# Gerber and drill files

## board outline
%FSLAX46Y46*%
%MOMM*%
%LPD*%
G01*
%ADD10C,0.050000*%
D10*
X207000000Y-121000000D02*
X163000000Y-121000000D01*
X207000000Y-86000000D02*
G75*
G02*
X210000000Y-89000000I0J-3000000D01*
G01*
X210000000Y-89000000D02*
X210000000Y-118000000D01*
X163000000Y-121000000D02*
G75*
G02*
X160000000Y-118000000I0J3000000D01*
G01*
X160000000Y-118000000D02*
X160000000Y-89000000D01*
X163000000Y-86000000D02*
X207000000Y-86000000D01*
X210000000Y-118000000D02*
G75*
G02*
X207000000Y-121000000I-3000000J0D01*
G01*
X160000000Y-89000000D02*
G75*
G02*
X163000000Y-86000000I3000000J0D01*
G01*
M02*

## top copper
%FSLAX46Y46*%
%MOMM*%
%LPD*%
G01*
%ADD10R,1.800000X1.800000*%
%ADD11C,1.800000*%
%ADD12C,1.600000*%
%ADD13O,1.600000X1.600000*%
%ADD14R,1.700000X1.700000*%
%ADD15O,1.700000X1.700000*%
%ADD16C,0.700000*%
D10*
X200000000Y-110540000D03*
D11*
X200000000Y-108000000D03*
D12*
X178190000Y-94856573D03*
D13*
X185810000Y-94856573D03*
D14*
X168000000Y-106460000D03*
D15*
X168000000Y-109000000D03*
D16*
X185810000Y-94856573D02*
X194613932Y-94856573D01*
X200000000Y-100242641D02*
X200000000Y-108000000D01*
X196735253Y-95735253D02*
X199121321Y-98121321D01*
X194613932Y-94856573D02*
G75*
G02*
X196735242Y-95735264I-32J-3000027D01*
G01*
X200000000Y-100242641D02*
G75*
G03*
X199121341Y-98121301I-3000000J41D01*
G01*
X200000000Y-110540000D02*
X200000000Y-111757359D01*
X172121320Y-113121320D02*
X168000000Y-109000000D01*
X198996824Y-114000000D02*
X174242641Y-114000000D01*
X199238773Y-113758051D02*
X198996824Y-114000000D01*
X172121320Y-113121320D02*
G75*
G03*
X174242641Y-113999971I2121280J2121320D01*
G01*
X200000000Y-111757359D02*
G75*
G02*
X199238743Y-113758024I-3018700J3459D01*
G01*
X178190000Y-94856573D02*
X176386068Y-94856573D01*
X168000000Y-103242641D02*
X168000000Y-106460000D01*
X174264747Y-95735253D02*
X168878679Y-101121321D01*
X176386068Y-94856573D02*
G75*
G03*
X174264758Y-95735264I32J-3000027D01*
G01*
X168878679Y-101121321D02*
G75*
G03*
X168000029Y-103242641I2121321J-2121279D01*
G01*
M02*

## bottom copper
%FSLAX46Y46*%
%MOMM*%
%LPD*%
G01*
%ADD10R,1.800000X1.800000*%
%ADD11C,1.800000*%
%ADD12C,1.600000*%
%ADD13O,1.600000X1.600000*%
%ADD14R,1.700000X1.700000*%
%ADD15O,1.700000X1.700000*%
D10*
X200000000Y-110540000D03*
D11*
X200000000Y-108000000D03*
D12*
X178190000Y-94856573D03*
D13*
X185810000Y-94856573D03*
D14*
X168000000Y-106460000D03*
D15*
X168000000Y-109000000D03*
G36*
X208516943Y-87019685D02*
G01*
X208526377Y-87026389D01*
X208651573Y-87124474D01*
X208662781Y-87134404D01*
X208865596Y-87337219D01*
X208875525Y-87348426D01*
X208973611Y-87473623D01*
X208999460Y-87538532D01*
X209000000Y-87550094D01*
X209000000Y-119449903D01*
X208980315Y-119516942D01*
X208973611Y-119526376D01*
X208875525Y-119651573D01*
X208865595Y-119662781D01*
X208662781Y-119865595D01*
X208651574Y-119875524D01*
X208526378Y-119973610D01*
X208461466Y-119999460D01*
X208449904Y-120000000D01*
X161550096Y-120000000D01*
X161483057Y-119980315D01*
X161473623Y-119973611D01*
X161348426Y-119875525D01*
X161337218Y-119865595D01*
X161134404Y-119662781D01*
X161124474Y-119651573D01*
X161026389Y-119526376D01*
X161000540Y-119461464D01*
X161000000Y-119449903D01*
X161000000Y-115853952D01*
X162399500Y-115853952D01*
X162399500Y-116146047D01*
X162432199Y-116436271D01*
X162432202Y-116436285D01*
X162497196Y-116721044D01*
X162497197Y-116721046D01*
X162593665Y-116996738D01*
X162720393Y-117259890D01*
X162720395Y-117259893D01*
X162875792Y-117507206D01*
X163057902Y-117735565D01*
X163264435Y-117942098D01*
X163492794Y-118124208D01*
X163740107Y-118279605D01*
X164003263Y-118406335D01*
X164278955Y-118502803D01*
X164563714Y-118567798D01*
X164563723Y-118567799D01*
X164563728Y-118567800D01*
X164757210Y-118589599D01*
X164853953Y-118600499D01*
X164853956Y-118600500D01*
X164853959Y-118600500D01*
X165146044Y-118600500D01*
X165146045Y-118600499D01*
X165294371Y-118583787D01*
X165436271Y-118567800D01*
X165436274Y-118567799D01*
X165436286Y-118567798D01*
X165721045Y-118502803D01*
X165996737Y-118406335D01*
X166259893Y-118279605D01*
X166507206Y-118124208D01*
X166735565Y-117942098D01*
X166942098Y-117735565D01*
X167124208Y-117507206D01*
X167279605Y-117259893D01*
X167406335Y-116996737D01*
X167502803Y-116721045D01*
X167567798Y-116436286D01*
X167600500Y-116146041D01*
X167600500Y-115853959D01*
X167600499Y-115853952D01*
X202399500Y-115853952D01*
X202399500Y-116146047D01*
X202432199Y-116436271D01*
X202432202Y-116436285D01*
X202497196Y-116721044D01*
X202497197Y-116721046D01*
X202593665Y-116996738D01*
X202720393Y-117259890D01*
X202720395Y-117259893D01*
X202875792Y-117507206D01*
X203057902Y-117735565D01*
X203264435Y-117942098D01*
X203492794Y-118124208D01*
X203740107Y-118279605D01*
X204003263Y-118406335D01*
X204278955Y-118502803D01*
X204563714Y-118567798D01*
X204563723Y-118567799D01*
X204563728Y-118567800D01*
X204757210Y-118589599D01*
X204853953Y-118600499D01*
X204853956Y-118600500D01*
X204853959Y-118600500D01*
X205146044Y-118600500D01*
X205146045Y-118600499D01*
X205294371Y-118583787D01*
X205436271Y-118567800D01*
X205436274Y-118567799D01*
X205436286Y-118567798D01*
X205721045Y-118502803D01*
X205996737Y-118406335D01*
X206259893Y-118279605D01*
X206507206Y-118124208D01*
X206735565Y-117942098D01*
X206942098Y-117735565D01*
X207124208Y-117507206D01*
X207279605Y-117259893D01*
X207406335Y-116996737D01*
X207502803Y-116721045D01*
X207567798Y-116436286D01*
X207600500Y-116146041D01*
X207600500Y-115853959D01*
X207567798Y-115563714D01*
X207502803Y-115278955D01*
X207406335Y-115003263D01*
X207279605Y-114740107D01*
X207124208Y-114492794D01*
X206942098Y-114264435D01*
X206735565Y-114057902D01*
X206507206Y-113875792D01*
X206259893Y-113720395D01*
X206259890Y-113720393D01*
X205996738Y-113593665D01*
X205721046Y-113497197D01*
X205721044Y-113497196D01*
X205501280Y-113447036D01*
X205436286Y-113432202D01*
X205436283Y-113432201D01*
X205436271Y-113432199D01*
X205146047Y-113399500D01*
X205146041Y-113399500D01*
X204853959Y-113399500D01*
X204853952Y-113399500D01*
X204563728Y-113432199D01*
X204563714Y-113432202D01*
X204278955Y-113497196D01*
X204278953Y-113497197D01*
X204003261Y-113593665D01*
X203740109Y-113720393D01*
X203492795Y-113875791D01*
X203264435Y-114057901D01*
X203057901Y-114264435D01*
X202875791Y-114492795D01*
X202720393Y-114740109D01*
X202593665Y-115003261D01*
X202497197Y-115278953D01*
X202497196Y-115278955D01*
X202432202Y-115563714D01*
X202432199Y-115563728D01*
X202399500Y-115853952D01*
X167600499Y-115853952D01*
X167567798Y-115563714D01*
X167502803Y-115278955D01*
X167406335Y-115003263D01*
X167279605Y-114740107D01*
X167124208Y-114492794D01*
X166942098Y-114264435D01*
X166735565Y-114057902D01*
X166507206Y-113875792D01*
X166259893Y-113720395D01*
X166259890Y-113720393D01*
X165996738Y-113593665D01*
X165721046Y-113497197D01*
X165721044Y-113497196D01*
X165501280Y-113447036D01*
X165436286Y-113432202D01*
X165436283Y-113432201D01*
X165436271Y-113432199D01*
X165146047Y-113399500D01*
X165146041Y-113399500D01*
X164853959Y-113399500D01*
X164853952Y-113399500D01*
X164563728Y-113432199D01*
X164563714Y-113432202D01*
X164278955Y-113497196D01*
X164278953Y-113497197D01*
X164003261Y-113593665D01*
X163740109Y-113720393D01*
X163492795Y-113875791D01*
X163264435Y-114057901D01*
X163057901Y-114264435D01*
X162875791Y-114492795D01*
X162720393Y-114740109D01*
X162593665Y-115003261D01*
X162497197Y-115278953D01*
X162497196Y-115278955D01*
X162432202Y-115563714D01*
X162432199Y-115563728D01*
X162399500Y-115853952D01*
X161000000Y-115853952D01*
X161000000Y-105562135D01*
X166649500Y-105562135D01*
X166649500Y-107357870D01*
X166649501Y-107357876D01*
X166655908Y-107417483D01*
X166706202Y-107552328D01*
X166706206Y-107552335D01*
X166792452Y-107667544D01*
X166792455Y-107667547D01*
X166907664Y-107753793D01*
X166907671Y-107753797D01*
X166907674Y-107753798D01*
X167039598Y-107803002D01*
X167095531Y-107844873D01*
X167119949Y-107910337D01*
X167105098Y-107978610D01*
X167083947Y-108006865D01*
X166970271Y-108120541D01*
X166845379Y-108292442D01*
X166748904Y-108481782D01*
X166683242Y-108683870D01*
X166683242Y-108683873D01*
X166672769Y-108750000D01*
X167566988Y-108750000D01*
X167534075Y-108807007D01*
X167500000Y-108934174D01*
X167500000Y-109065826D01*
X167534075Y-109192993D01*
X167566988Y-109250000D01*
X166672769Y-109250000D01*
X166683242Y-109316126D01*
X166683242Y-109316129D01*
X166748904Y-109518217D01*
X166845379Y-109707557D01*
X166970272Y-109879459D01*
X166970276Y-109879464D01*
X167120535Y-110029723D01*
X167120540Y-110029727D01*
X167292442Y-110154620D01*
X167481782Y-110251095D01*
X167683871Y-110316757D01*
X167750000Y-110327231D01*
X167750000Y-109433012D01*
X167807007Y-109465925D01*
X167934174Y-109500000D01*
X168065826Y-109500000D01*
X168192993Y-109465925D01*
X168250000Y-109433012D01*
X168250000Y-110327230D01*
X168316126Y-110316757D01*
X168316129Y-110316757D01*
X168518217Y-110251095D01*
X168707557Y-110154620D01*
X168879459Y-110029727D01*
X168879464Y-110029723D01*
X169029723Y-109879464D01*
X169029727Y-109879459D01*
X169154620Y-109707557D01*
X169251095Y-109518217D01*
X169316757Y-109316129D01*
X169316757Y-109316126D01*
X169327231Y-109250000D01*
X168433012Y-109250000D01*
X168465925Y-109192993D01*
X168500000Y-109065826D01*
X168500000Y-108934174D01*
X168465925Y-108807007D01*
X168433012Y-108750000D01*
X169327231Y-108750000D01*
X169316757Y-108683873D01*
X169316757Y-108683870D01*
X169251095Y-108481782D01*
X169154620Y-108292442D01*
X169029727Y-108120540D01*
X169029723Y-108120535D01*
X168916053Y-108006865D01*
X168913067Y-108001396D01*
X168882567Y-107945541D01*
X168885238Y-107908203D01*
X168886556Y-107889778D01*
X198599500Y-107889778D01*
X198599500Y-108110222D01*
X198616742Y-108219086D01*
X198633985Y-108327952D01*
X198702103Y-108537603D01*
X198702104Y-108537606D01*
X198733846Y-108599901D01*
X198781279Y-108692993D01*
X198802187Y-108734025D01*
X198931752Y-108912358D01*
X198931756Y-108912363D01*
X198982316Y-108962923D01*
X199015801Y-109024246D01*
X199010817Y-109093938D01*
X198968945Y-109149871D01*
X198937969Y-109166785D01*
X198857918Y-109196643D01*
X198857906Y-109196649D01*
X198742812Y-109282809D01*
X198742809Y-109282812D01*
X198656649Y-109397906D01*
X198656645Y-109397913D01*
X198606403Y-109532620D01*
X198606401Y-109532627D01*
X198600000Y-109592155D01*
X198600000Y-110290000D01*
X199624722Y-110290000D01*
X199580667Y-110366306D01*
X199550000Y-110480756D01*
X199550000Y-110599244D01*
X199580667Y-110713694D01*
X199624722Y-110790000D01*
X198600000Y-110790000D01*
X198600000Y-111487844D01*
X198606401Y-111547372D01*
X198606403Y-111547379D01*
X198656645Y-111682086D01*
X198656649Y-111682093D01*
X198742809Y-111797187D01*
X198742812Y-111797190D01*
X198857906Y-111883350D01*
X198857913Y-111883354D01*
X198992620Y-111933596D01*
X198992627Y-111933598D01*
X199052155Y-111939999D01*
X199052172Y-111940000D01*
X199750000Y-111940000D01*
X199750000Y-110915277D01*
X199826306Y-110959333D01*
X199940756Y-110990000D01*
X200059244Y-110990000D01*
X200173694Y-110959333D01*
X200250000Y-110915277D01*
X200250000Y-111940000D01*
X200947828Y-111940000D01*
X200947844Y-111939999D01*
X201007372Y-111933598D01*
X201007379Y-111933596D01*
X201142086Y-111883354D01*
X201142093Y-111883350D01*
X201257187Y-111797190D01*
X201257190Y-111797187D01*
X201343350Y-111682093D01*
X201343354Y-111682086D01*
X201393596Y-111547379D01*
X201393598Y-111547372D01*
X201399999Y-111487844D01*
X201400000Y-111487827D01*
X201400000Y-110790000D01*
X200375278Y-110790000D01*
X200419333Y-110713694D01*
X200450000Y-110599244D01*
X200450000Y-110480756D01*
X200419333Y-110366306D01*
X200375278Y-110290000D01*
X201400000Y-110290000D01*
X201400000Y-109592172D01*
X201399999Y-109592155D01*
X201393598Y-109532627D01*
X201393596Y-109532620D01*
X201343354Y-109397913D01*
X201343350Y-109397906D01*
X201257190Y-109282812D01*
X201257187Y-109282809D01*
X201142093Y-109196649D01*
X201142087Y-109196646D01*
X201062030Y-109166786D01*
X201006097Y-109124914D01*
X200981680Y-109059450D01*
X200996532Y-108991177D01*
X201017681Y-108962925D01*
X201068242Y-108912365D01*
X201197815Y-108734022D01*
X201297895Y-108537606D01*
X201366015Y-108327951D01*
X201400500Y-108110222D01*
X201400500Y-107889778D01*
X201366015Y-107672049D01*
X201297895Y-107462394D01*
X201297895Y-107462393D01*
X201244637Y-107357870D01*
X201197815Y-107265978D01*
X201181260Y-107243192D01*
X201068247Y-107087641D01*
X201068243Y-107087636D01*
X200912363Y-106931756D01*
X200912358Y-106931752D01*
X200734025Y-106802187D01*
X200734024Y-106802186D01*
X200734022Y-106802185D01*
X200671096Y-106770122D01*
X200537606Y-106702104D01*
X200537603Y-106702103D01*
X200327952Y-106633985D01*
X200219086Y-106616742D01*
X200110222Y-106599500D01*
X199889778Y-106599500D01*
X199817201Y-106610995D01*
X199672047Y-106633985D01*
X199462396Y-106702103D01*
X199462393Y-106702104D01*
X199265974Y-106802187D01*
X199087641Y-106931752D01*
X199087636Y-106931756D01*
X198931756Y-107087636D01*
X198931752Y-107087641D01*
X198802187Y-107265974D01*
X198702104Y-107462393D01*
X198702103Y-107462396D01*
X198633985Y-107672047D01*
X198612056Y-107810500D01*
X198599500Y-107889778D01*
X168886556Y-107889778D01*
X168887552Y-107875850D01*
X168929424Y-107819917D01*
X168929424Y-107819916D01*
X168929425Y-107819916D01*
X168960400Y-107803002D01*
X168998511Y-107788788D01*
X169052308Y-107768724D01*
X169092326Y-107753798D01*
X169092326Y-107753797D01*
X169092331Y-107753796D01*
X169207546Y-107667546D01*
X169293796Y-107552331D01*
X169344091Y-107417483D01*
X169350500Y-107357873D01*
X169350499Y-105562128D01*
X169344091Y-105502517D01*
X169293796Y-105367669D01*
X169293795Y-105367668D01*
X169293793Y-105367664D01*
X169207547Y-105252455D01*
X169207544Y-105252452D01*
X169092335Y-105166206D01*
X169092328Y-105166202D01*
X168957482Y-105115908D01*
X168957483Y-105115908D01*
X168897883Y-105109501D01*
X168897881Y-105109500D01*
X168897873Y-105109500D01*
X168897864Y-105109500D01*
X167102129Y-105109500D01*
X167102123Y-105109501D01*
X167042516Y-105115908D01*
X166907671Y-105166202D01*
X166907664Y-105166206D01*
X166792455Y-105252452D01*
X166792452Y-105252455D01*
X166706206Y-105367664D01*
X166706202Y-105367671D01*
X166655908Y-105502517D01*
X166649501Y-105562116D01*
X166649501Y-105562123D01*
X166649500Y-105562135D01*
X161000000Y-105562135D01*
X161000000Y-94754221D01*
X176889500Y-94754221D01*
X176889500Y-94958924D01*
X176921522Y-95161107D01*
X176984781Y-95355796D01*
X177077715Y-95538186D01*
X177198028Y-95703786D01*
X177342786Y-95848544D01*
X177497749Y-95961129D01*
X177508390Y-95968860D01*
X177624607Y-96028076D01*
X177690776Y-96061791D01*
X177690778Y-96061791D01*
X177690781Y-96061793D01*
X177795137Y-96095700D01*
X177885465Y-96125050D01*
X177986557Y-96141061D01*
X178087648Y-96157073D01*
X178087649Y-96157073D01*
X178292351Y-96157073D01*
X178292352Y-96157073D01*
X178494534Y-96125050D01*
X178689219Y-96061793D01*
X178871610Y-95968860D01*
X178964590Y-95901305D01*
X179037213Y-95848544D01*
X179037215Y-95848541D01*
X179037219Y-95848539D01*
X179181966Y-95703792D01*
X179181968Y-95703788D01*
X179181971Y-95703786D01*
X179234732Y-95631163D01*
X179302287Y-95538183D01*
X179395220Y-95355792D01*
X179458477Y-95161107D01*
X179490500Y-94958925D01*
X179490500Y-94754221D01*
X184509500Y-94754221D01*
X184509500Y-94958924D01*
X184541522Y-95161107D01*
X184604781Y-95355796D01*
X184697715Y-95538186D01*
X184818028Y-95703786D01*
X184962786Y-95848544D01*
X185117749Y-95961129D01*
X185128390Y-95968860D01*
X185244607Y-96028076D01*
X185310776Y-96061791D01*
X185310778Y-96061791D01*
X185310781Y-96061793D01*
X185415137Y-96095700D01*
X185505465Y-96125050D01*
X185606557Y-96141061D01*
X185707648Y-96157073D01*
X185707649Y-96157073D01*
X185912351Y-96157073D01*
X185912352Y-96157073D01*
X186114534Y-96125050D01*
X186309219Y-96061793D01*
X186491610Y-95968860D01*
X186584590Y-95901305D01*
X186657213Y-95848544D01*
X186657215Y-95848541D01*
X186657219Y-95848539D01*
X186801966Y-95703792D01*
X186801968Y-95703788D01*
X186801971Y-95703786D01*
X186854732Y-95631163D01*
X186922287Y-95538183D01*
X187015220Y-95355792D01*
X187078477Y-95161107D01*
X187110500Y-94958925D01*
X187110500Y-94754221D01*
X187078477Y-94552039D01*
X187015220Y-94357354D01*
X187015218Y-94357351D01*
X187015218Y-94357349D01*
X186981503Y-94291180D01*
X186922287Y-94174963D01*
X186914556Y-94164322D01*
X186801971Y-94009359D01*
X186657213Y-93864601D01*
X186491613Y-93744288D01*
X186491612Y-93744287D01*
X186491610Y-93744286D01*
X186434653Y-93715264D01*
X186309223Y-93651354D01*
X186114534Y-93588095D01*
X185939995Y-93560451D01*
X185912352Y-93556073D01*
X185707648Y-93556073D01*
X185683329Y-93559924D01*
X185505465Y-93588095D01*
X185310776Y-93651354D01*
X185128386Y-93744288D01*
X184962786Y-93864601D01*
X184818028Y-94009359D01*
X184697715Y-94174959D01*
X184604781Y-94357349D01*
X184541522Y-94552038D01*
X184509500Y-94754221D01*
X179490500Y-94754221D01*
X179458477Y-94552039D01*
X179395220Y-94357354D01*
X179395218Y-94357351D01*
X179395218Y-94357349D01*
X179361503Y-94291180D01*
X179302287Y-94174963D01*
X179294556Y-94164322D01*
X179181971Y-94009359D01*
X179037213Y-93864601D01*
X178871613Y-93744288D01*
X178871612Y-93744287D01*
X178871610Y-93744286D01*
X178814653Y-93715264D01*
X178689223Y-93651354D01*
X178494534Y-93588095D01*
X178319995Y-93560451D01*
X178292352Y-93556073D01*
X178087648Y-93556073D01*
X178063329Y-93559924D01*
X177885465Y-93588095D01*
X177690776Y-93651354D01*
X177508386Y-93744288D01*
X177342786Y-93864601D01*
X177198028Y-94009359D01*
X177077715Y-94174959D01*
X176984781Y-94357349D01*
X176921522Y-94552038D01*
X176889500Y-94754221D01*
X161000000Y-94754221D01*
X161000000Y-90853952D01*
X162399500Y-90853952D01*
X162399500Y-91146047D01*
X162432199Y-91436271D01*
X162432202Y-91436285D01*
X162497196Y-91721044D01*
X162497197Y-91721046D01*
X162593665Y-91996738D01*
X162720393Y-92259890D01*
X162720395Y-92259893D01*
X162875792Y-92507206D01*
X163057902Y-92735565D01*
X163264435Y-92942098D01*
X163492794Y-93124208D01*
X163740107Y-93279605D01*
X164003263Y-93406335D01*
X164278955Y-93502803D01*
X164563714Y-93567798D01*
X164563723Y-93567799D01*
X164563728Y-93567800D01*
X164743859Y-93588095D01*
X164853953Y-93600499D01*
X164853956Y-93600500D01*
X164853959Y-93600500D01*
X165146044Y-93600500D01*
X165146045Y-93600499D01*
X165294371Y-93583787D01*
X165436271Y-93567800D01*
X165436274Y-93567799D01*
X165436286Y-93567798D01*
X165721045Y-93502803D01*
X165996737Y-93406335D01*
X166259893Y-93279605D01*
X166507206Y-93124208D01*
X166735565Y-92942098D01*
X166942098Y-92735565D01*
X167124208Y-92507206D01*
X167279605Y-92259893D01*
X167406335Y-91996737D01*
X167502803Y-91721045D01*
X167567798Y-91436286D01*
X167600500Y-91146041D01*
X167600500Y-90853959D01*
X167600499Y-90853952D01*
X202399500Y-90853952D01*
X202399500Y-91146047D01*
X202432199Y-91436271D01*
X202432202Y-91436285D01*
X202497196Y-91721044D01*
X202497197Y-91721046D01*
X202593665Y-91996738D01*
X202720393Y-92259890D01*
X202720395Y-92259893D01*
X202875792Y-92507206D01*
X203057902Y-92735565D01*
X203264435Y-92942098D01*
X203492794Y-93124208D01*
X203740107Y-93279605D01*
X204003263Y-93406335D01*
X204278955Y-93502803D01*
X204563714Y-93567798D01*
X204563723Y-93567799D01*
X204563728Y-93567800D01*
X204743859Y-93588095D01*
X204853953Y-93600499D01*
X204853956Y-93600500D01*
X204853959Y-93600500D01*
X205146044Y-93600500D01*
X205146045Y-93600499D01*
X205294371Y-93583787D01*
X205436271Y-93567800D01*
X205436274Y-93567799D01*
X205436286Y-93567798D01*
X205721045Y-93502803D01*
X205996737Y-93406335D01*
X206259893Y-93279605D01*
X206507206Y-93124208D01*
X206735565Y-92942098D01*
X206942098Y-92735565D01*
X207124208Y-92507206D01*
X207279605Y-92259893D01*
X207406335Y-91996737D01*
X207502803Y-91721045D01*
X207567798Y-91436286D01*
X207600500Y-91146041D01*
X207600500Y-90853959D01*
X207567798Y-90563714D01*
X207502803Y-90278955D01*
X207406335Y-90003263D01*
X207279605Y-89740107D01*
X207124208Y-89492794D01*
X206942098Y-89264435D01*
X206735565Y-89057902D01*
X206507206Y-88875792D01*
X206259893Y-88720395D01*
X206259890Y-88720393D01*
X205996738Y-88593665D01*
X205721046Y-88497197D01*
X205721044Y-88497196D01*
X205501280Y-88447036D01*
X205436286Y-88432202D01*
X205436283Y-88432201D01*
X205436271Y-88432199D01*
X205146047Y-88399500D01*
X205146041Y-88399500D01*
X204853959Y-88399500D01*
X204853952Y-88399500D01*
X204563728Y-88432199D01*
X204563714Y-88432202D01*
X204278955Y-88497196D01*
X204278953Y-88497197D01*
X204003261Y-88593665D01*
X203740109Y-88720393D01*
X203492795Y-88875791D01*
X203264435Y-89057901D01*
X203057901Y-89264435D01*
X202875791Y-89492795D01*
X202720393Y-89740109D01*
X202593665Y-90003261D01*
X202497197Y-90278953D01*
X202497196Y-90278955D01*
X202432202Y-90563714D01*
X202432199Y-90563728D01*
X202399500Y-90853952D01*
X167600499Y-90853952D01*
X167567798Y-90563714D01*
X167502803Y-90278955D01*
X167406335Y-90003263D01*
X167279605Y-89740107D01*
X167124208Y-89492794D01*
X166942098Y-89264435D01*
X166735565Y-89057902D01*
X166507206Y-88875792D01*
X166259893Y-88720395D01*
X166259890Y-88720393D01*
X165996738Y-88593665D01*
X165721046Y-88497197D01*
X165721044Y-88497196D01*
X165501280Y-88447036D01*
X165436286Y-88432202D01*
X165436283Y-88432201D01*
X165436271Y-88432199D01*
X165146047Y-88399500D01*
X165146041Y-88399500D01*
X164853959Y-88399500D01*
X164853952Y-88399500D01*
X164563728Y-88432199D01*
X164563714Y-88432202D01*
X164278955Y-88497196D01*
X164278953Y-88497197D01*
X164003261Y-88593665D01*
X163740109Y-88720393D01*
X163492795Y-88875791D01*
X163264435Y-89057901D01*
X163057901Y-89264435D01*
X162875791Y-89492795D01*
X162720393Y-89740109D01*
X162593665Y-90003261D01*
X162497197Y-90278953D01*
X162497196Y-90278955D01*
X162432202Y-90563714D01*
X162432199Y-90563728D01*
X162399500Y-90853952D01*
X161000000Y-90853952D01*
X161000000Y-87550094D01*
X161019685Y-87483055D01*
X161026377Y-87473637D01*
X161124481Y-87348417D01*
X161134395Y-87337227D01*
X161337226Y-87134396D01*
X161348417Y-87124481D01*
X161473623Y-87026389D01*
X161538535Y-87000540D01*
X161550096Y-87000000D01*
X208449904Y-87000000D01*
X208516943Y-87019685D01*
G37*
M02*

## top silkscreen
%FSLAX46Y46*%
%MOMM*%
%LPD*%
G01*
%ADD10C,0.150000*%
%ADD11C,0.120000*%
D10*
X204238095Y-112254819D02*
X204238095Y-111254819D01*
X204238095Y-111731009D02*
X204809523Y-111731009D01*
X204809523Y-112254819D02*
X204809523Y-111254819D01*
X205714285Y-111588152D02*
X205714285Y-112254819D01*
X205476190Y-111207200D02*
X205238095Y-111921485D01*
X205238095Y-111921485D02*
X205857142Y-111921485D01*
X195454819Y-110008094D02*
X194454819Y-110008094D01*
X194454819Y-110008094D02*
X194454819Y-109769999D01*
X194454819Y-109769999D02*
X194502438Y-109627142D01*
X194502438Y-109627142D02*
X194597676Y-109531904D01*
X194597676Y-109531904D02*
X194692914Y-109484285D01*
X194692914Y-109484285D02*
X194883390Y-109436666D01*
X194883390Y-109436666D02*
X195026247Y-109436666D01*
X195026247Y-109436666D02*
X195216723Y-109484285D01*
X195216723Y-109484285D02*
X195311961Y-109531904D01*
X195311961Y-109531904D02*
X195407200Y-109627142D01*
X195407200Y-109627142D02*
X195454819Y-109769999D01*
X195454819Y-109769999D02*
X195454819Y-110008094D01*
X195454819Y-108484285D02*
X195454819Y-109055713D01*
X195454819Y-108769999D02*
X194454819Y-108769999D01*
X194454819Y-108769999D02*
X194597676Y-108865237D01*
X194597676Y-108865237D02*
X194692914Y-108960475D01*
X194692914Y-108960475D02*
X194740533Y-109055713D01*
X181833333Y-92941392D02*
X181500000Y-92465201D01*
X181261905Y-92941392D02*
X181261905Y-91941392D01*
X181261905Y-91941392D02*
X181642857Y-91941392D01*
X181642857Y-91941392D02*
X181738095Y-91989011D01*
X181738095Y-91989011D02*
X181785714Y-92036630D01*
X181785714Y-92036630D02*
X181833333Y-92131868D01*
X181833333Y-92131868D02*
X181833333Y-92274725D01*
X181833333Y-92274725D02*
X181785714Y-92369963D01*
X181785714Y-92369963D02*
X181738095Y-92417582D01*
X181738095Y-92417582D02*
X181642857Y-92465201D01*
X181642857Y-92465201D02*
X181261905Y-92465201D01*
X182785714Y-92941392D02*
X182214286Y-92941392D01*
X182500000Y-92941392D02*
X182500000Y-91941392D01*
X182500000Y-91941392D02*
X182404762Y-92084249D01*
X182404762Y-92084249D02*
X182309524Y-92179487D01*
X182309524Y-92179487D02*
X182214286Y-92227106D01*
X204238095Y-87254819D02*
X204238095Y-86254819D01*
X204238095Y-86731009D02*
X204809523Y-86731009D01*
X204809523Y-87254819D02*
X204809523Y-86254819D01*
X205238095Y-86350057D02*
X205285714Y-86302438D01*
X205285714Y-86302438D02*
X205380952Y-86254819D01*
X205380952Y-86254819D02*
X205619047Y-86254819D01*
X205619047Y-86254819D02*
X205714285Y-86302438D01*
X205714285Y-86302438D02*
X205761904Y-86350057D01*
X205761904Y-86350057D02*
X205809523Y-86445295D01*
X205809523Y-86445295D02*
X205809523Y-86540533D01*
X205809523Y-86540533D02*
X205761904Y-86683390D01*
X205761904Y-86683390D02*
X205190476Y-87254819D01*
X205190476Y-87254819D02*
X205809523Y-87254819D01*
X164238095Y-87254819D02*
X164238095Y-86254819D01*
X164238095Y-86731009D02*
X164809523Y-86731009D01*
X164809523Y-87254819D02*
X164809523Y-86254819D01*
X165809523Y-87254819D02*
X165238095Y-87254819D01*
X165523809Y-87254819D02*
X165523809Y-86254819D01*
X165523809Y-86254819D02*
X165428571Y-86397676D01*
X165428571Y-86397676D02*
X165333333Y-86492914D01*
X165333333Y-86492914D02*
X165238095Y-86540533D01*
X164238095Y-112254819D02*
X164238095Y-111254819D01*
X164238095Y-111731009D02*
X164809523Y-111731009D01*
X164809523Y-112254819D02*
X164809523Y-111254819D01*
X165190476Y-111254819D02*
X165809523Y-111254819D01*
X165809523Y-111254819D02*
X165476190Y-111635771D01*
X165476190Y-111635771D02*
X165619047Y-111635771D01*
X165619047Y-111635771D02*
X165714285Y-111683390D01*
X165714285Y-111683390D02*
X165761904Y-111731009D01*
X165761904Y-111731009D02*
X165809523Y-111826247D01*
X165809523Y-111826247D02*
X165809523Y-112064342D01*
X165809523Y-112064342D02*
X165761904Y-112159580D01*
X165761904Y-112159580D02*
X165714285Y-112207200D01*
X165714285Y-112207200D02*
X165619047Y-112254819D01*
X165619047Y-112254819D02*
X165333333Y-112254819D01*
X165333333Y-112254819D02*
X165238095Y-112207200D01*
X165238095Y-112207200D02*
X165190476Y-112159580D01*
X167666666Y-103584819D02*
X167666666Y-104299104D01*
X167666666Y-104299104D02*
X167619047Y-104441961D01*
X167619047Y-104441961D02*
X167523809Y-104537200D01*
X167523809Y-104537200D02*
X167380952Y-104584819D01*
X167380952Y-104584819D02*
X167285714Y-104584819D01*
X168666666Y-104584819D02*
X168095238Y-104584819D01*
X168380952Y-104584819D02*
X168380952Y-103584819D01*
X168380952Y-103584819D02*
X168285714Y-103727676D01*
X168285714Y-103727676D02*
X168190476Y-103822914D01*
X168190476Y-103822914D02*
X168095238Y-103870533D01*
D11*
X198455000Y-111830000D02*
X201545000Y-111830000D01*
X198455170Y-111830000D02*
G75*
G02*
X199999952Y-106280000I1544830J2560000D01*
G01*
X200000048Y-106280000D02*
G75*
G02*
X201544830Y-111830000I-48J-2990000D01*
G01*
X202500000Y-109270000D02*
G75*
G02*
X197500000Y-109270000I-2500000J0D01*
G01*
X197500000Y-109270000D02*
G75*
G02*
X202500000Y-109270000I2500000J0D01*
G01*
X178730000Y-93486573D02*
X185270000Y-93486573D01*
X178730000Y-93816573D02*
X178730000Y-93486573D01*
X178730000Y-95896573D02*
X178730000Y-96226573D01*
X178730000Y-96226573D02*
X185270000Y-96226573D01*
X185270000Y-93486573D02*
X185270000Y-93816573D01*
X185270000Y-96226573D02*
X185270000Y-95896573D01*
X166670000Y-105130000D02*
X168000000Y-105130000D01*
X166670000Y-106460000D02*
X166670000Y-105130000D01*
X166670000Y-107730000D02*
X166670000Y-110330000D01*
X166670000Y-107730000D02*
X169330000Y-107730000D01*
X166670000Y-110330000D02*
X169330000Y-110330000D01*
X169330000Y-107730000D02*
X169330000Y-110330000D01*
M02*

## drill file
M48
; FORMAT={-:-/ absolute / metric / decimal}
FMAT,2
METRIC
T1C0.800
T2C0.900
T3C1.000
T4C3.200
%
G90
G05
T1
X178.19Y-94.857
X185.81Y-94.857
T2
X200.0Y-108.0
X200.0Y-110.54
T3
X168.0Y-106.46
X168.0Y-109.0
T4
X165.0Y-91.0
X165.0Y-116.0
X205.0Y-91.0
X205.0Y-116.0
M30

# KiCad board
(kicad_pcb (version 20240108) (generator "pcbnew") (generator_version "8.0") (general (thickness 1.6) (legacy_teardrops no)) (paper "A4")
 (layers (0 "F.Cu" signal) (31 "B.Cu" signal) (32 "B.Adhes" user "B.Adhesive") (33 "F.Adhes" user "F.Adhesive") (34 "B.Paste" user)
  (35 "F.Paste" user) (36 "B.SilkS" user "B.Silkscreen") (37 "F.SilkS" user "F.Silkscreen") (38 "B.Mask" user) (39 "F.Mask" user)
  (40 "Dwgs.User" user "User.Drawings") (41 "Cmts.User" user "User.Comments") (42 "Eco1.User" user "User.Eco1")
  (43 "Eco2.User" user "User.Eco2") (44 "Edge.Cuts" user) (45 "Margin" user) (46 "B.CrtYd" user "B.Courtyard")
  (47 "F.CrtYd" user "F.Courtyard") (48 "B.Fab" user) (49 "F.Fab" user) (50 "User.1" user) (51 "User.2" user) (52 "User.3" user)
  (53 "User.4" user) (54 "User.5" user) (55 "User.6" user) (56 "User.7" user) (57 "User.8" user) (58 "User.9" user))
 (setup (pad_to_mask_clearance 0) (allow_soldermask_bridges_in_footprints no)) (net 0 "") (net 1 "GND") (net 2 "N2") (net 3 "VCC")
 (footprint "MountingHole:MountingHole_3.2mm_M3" (layer "F.Cu") (at 205 116)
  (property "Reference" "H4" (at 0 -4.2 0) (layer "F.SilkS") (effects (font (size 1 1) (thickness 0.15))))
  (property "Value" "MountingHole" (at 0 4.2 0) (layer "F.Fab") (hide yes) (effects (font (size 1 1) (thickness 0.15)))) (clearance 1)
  (pad "" np_thru_hole circle (at 0 0) (size 3.2 3.2) (drill 3.2) (layers "*.Cu" "*.Mask")))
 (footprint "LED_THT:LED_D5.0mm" (layer "F.Cu") (at 200 110.54 90)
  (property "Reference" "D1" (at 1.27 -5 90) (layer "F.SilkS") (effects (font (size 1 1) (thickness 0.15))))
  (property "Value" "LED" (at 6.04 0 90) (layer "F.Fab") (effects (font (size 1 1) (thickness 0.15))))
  (fp_line (start -1.29 -1.545) (end -1.29 1.545) (stroke (width 0.12) (type solid)) (layer "F.SilkS"))
  (fp_arc (start -1.29 -1.54483) (mid 2.071756 -2.880501) (end 4.26 -0.000048) (stroke (width 0.12) (type solid)) (layer "F.SilkS"))
  (fp_arc (start 4.26 0.000048) (mid 2.071756 2.880501) (end -1.29 1.54483) (stroke (width 0.12) (type solid)) (layer "F.SilkS"))
  (fp_circle (center 1.27 0) (end 3.77 0) (stroke (width 0.12) (type solid)) (fill none) (layer "F.SilkS"))
  (pad "1" thru_hole rect (at 0 0 90) (size 1.8 1.8) (drill 0.9) (layers "*.Cu" "*.Mask") (remove_unused_layers no) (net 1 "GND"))
  (pad "2" thru_hole circle (at 2.54 0 90) (size 1.8 1.8) (drill 0.9) (layers "*.Cu" "*.Mask") (remove_unused_layers no) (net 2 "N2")))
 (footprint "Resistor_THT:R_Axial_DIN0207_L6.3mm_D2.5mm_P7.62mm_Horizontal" (layer "F.Cu") (at 178.19 94.856573)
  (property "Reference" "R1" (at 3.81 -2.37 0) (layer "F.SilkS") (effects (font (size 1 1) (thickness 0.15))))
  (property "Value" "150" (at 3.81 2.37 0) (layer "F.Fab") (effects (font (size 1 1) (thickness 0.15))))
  (fp_line (start 0.54 -1.37) (end 7.08 -1.37) (stroke (width 0.12) (type solid)) (layer "F.SilkS"))
  (fp_line (start 0.54 -1.04) (end 0.54 -1.37) (stroke (width 0.12) (type solid)) (layer "F.SilkS"))
  (fp_line (start 0.54 1.04) (end 0.54 1.37) (stroke (width 0.12) (type solid)) (layer "F.SilkS"))
  (fp_line (start 0.54 1.37) (end 7.08 1.37) (stroke (width 0.12) (type solid)) (layer "F.SilkS"))
  (fp_line (start 7.08 -1.37) (end 7.08 -1.04) (stroke (width 0.12) (type solid)) (layer "F.SilkS"))
  (fp_line (start 7.08 1.37) (end 7.08 1.04) (stroke (width 0.12) (type solid)) (layer "F.SilkS"))
  (pad "1" thru_hole circle (at 0 0) (size 1.6 1.6) (drill 0.8) (layers "*.Cu" "*.Mask") (remove_unused_layers no) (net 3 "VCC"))
  (pad "2" thru_hole oval (at 7.62 0) (size 1.6 1.6) (drill 0.8) (layers "*.Cu" "*.Mask") (remove_unused_layers no) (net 2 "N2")))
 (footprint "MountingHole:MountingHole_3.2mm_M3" (layer "F.Cu") (at 205 91)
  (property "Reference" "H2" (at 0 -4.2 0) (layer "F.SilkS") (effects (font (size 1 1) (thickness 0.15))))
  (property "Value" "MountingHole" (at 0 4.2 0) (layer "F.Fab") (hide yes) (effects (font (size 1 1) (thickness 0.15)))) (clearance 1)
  (pad "" np_thru_hole circle (at 0 0) (size 3.2 3.2) (drill 3.2) (layers "*.Cu" "*.Mask")))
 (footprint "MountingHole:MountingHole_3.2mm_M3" (layer "F.Cu") (at 165 91)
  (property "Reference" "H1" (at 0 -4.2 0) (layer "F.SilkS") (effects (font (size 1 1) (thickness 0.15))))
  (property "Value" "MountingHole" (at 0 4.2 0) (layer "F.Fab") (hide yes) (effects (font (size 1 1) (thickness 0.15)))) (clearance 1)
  (pad "" np_thru_hole circle (at 0 0) (size 3.2 3.2) (drill 3.2) (layers "*.Cu" "*.Mask")))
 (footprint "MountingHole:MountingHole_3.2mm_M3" (layer "F.Cu") (at 165 116)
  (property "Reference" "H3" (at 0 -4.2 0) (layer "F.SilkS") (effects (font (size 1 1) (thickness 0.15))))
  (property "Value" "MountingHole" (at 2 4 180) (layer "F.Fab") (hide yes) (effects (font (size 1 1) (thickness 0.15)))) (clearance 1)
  (pad "" np_thru_hole circle (at 0 0) (size 3.2 3.2) (drill 3.2) (layers "*.Cu" "*.Mask")))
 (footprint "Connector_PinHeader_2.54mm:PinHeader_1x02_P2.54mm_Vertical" (layer "F.Cu") (at 168 106.46)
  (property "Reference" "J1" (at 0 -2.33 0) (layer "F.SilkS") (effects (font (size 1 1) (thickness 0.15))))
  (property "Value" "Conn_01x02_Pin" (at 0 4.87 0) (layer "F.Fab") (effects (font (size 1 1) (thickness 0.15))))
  (fp_line (start -1.33 -1.33) (end 0 -1.33) (stroke (width 0.12) (type solid)) (layer "F.SilkS"))
  (fp_line (start -1.33 0) (end -1.33 -1.33) (stroke (width 0.12) (type solid)) (layer "F.SilkS"))
  (fp_line (start -1.33 1.27) (end -1.33 3.87) (stroke (width 0.12) (type solid)) (layer "F.SilkS"))
  (fp_line (start -1.33 1.27) (end 1.33 1.27) (stroke (width 0.12) (type solid)) (layer "F.SilkS"))
  (fp_line (start -1.33 3.87) (end 1.33 3.87) (stroke (width 0.12) (type solid)) (layer "F.SilkS"))
  (fp_line (start 1.33 1.27) (end 1.33 3.87) (stroke (width 0.12) (type solid)) (layer "F.SilkS"))
  (pad "1" thru_hole rect (at 0 0) (size 1.7 1.7) (drill 1) (layers "*.Cu" "*.Mask") (remove_unused_layers no) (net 3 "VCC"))
  (pad "2" thru_hole oval (at 0 2.54) (size 1.7 1.7) (drill 1) (layers "*.Cu" "*.Mask") (remove_unused_layers no) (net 1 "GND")))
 (gr_line (start 207 121) (end 163 121) (stroke (width 0.05) (type default)) (layer "Edge.Cuts"))
 (gr_arc (start 207 86) (mid 209.12132 86.87868) (end 210 89) (stroke (width 0.05) (type default)) (layer "Edge.Cuts"))
 (gr_line (start 210 89) (end 210 118) (stroke (width 0.05) (type default)) (layer "Edge.Cuts"))
 (gr_arc (start 163 121) (mid 160.87868 120.12132) (end 160 118) (stroke (width 0.05) (type default)) (layer "Edge.Cuts"))
 (gr_line (start 160 118) (end 160 89) (stroke (width 0.05) (type default)) (layer "Edge.Cuts"))
 (gr_line (start 163 86) (end 207 86) (stroke (width 0.05) (type default)) (layer "Edge.Cuts"))
 (gr_arc (start 210 118) (mid 209.12132 120.12132) (end 207 121) (stroke (width 0.05) (type default)) (layer "Edge.Cuts"))
 (gr_arc (start 160 89) (mid 160.87868 86.87868) (end 163 86) (stroke (width 0.05) (type default)) (layer "Edge.Cuts"))
 (segment (start 185.81 94.856573) (end 194.613932 94.856573) (width 0.7) (layer "F.Cu") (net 2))
 (segment (start 200 100.242641) (end 200 108) (width 0.7) (layer "F.Cu") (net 2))
 (segment (start 196.735253 95.735253) (end 199.121321 98.121321) (width 0.7) (layer "F.Cu") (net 2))
 (arc (start 194.613932 94.856573) (mid 195.761983 95.084935) (end 196.735253 95.735253) (width 0.7) (layer "F.Cu") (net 2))
 (arc (start 200 100.242641) (mid 199.771639 99.094591) (end 199.121321 98.121321) (width 0.7) (layer "F.Cu") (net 2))
 (segment (start 200 110.54) (end 200 111.757359) (width 0.7) (layer "F.Cu") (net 1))
 (segment (start 172.12132 113.12132) (end 168 109) (width 0.7) (layer "F.Cu") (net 1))
 (segment (start 198.996824 114) (end 174.242641 114) (width 0.7) (layer "F.Cu") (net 1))
 (segment (start 199.238773 113.758051) (end 198.996824 114) (width 0.7) (layer "F.Cu") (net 1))
 (arc (start 172.12132 113.12132) (mid 173.09459 113.771639) (end 174.242641 114) (width 0.7) (layer "F.Cu") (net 1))
 (arc (start 200 111.757359) (mid 199.802759 112.827232) (end 199.238773 113.758051) (width 0.7) (layer "F.Cu") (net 1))
 (segment (start 178.19 94.856573) (end 176.386068 94.856573) (width 0.7) (layer "F.Cu") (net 3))
 (segment (start 168 103.242641) (end 168 106.46) (width 0.7) (layer "F.Cu") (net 3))
 (segment (start 174.264747 95.735253) (end 168.878679 101.121321) (width 0.7) (layer "F.Cu") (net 3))
 (arc (start 176.386068 94.856573) (mid 175.238017 95.084935) (end 174.264747 95.735253) (width 0.7) (layer "F.Cu") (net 3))
 (arc (start 168.878679 101.121321) (mid 168.228361 102.094591) (end 168 103.242641) (width 0.7) (layer "F.Cu") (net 3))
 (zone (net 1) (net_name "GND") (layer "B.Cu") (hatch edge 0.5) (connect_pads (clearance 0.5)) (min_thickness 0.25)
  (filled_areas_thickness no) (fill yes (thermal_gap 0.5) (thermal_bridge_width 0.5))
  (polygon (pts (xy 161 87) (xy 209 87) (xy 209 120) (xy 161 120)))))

